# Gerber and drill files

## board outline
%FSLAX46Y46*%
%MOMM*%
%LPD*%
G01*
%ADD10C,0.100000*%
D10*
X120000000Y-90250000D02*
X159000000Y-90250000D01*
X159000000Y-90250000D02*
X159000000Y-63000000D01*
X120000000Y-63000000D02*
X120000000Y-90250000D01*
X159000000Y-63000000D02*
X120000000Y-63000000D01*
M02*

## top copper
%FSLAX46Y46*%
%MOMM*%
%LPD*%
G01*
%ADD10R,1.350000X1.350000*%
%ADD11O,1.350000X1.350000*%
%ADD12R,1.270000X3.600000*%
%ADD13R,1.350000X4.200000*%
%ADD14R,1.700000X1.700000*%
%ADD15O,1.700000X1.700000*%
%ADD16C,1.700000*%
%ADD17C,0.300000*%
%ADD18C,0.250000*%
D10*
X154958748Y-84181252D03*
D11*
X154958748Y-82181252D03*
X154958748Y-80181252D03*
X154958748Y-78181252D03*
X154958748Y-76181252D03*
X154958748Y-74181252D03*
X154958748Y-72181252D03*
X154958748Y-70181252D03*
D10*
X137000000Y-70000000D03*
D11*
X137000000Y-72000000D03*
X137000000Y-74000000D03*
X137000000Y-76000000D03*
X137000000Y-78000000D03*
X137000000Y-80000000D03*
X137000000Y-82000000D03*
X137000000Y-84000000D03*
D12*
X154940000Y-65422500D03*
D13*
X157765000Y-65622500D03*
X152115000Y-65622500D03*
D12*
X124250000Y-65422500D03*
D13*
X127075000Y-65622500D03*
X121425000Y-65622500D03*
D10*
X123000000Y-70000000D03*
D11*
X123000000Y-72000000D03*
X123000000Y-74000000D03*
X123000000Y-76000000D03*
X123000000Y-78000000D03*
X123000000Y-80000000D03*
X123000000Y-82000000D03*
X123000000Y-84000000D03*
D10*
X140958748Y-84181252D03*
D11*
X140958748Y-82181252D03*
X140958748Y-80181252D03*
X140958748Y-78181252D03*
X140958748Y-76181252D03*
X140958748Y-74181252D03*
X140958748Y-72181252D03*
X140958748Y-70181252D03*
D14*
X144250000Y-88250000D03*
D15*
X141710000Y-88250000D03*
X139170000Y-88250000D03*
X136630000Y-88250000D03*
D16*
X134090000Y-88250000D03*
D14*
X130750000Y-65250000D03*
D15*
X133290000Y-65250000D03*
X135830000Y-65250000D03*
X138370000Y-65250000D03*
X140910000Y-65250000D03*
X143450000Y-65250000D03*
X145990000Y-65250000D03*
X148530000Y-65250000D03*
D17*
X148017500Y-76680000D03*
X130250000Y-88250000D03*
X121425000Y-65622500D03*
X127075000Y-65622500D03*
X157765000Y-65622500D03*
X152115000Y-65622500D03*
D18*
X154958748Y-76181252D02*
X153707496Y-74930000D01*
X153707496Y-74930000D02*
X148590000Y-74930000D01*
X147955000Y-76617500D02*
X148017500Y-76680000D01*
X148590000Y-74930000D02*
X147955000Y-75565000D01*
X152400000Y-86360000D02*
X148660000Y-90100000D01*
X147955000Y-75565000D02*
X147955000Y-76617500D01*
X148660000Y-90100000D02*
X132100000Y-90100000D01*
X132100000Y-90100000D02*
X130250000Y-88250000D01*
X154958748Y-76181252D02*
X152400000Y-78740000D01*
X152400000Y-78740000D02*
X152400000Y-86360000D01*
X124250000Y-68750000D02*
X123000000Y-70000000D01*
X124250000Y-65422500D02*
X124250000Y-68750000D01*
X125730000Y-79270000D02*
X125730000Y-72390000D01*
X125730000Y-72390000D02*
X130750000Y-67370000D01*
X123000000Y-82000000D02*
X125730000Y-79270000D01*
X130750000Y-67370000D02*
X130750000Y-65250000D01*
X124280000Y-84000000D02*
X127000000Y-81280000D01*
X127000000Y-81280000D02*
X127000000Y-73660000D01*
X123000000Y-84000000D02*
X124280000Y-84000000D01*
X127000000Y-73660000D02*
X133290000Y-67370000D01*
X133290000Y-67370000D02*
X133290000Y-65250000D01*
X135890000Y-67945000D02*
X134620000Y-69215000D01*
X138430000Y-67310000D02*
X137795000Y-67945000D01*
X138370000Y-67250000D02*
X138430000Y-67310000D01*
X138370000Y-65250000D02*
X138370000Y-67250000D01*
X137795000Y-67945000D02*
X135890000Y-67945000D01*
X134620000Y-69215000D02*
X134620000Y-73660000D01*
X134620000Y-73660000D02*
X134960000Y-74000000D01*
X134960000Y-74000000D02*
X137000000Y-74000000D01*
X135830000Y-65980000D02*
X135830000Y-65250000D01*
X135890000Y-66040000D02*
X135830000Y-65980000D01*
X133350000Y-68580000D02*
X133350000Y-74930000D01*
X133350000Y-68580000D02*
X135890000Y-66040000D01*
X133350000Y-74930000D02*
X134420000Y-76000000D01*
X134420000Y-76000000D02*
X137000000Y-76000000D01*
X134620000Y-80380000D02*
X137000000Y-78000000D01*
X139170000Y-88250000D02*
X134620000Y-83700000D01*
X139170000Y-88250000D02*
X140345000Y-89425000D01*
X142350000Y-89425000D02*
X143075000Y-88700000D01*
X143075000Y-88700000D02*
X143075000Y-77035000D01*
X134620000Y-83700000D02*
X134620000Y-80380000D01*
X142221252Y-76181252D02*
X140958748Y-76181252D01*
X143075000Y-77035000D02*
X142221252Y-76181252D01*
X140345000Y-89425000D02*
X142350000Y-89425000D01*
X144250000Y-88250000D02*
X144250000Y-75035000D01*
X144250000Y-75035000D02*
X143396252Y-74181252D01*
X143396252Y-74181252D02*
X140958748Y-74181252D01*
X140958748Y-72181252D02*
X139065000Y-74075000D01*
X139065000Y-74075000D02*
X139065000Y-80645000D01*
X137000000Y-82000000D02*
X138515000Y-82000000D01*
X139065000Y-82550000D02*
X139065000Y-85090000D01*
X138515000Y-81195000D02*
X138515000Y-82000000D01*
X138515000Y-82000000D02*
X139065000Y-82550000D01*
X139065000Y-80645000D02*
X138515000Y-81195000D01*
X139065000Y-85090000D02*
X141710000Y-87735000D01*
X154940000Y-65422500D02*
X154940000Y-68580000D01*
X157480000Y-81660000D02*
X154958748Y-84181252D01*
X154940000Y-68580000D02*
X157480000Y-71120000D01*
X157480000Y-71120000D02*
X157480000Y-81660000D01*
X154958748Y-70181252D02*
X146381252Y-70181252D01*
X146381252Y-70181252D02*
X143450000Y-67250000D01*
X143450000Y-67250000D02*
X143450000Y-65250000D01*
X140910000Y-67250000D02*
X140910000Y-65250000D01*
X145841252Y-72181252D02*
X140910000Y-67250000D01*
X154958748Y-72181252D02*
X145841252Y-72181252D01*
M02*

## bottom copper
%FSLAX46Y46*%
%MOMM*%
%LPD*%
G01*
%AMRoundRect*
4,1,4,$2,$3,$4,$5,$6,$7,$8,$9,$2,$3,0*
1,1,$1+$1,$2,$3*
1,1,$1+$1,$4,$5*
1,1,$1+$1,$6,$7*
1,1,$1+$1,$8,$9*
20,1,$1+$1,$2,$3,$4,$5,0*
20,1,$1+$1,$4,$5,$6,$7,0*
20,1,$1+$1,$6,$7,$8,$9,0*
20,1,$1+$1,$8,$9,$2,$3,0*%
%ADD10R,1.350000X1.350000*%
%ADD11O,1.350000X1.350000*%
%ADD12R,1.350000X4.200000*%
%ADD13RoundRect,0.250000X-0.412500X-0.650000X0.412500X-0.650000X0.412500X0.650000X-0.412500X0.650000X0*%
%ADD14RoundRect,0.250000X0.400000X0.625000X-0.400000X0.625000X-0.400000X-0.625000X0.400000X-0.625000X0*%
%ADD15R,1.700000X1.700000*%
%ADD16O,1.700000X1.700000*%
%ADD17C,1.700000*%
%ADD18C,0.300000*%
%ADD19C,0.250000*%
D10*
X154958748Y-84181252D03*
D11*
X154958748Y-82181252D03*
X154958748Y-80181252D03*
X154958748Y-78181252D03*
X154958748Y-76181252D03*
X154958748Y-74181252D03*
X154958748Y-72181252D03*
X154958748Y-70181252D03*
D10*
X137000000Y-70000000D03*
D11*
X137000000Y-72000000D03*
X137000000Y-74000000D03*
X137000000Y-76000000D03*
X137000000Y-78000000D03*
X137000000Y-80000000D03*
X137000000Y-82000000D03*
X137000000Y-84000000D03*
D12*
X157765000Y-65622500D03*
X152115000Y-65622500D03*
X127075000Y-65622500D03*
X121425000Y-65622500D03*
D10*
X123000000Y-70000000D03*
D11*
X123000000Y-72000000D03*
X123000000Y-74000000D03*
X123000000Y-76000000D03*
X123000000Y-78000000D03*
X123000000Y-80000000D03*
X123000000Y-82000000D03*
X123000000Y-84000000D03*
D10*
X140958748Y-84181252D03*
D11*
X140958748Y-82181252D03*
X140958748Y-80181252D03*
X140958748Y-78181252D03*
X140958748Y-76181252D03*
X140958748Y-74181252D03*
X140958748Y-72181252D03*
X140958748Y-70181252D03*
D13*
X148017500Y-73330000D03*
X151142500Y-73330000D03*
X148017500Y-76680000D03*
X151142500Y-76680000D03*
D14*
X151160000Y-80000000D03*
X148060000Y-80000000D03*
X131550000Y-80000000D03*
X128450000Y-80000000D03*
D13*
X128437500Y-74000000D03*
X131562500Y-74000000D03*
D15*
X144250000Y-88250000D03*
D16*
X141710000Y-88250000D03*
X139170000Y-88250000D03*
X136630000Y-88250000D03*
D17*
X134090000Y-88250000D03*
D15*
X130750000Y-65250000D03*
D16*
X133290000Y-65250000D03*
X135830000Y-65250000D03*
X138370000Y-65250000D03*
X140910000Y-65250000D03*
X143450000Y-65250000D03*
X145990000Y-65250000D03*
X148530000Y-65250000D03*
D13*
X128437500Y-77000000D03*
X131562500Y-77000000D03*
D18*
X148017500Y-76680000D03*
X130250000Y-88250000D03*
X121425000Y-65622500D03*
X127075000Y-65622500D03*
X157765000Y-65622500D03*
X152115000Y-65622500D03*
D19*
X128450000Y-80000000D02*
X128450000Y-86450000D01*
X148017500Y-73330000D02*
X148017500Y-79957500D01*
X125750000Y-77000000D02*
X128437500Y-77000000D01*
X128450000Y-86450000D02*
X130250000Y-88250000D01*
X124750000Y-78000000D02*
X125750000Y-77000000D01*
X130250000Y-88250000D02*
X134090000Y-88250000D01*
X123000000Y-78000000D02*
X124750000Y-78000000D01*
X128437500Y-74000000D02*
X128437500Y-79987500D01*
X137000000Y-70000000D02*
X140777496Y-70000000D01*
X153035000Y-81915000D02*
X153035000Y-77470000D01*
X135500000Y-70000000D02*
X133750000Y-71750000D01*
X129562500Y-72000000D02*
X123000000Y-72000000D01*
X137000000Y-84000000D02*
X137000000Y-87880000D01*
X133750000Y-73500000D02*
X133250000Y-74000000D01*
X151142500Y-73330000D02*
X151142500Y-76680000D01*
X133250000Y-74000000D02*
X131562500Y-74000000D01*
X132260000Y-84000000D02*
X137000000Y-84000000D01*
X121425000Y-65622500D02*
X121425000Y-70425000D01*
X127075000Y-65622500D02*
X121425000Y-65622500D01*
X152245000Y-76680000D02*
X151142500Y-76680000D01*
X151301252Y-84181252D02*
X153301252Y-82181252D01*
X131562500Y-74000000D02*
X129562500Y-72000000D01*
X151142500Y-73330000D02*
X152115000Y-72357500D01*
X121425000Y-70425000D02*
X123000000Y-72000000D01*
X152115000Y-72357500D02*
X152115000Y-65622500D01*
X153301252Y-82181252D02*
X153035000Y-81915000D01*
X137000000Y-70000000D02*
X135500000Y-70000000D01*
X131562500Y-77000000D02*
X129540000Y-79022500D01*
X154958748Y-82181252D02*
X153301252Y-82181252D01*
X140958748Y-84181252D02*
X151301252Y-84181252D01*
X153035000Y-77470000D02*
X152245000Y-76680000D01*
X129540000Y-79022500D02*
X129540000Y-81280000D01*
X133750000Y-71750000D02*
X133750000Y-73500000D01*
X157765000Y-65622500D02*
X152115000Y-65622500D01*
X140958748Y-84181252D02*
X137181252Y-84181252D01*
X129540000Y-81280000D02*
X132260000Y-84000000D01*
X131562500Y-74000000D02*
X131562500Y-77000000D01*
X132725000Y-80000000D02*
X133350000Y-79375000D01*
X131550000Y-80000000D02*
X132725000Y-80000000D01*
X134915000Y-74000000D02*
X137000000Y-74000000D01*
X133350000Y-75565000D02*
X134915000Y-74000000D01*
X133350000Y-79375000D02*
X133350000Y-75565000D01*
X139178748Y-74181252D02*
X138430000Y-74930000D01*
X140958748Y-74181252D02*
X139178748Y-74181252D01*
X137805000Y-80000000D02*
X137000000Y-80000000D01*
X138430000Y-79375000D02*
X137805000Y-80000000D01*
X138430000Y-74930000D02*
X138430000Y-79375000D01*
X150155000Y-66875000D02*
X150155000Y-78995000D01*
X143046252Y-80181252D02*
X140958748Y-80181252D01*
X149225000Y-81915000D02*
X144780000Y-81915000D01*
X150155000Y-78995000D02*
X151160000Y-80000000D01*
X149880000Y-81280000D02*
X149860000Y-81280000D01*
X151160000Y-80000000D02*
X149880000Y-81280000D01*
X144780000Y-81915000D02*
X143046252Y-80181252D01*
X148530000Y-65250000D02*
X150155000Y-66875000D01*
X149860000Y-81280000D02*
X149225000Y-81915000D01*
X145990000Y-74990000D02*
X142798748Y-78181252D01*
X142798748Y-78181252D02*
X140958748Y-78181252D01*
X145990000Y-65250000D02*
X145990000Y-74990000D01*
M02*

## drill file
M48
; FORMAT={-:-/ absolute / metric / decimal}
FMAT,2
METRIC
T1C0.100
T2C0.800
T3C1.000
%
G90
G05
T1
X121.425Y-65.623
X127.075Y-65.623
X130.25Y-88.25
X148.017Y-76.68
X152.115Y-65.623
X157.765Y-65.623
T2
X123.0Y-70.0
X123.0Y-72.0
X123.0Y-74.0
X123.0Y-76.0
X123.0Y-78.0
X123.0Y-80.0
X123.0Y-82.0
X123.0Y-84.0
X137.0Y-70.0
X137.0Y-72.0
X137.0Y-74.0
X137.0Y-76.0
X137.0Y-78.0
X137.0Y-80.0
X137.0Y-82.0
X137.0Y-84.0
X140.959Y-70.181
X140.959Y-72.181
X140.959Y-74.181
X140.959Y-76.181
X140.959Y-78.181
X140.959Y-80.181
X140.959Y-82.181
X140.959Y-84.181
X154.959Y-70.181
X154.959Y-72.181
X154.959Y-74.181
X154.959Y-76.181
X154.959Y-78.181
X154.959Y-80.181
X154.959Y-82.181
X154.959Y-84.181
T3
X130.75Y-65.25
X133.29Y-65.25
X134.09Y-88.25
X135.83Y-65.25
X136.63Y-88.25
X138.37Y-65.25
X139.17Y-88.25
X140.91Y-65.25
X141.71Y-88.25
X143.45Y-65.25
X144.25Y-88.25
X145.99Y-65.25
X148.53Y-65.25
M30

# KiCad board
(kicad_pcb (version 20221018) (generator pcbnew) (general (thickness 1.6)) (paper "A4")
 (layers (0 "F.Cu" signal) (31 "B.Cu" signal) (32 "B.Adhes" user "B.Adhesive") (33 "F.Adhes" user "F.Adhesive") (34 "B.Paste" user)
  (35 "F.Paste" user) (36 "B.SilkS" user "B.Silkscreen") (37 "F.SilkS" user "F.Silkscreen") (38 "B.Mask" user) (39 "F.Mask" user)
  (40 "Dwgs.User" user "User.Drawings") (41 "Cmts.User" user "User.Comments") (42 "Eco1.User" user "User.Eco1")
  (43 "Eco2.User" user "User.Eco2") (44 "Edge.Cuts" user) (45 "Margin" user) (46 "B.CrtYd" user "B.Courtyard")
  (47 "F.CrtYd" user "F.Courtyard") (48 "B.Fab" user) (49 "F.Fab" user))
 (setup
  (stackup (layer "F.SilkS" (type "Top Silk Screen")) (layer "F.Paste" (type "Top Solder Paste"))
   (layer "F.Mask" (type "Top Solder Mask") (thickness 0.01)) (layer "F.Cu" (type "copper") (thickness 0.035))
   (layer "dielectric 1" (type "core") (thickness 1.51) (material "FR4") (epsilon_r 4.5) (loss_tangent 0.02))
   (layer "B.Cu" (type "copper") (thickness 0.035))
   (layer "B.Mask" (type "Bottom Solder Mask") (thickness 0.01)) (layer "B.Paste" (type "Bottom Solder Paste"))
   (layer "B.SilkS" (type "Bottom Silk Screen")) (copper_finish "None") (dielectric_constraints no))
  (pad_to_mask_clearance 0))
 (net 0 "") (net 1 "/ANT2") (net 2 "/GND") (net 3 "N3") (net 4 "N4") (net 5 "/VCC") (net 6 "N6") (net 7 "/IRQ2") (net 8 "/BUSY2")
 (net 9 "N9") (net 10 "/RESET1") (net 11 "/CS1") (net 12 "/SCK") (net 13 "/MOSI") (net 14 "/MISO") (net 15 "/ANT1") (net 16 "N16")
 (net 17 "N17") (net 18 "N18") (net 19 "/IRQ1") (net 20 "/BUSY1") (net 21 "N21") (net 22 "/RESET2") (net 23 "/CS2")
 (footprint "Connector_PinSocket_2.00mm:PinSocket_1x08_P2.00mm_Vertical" (layer "F.Cu") (at 154.958748 84.181252 180)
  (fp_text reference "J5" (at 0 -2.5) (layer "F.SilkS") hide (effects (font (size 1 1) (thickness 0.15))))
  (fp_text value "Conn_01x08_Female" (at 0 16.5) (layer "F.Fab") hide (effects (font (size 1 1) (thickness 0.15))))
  (pad "1" thru_hole rect (at 0 0 180) (size 1.35 1.35) (drill 0.8) (layers "*.Cu" "*.Mask") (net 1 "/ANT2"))
  (pad "2" thru_hole oval (at 0 2 180) (size 1.35 1.35) (drill 0.8) (layers "*.Cu" "*.Mask") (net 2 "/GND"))
  (pad "3" thru_hole oval (at 0 4 180) (size 1.35 1.35) (drill 0.8) (layers "*.Cu" "*.Mask") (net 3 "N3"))
  (pad "4" thru_hole oval (at 0 6 180) (size 1.35 1.35) (drill 0.8) (layers "*.Cu" "*.Mask") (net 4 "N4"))
  (pad "5" thru_hole oval (at 0 8 180) (size 1.35 1.35) (drill 0.8) (layers "*.Cu" "*.Mask") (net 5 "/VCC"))
  (pad "6" thru_hole oval (at 0 10 180) (size 1.35 1.35) (drill 0.8) (layers "*.Cu" "*.Mask") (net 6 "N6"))
  (pad "7" thru_hole oval (at 0 12 180) (size 1.35 1.35) (drill 0.8) (layers "*.Cu" "*.Mask") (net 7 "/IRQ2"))
  (pad "8" thru_hole oval (at 0 14 180) (size 1.35 1.35) (drill 0.8) (layers "*.Cu" "*.Mask") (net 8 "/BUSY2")))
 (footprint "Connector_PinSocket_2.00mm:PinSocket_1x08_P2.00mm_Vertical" (layer "F.Cu") (at 137 70)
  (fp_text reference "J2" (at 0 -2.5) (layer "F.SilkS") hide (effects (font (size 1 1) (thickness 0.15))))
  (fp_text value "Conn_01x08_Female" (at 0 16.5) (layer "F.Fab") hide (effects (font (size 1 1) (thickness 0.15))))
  (pad "1" thru_hole rect (at 0 0) (size 1.35 1.35) (drill 0.8) (layers "*.Cu" "*.Mask") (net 2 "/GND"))
  (pad "2" thru_hole oval (at 0 2) (size 1.35 1.35) (drill 0.8) (layers "*.Cu" "*.Mask") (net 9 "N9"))
  (pad "3" thru_hole oval (at 0 4) (size 1.35 1.35) (drill 0.8) (layers "*.Cu" "*.Mask") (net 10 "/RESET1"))
  (pad "4" thru_hole oval (at 0 6) (size 1.35 1.35) (drill 0.8) (layers "*.Cu" "*.Mask") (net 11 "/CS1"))
  (pad "5" thru_hole oval (at 0 8) (size 1.35 1.35) (drill 0.8) (layers "*.Cu" "*.Mask") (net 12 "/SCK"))
  (pad "6" thru_hole oval (at 0 10) (size 1.35 1.35) (drill 0.8) (layers "*.Cu" "*.Mask") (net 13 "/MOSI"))
  (pad "7" thru_hole oval (at 0 12) (size 1.35 1.35) (drill 0.8) (layers "*.Cu" "*.Mask") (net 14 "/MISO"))
  (pad "8" thru_hole oval (at 0 14) (size 1.35 1.35) (drill 0.8) (layers "*.Cu" "*.Mask") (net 2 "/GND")))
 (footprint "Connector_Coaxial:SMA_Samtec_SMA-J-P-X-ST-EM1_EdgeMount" (layer "F.Cu") (at 154.94 65.6225 180)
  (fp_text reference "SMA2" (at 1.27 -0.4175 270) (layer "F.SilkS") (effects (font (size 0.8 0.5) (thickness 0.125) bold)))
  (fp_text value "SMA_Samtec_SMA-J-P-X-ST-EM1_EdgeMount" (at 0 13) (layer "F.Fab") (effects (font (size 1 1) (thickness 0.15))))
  (pad "1" smd rect (at -2.825 0 180) (size 1.35 4.2) (layers "B.Cu" "B.Paste" "B.Mask") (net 2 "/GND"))
  (pad "1" smd rect (at 0 0.2 180) (size 1.27 3.6) (layers "F.Cu" "F.Paste" "F.Mask") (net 1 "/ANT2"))
  (pad "1" smd rect (at 2.825 0 180) (size 1.35 4.2) (layers "B.Cu" "B.Paste" "B.Mask") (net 2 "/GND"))
  (pad "2" smd rect (at -2.825 0 180) (size 1.35 4.2) (layers "F.Cu" "F.Paste" "F.Mask") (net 2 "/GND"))
  (pad "2" smd rect (at 2.825 0 180) (size 1.35 4.2) (layers "F.Cu" "F.Paste" "F.Mask") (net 2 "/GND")))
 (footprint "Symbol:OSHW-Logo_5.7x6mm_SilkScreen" (layer "F.Cu") (at 149 86.5)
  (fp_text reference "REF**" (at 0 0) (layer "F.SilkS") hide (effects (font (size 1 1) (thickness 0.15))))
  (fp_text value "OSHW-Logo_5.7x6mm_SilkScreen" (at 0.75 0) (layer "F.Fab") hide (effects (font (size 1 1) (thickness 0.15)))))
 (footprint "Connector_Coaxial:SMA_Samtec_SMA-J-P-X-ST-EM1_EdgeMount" (layer "F.Cu") (at 124.25 65.6225 180)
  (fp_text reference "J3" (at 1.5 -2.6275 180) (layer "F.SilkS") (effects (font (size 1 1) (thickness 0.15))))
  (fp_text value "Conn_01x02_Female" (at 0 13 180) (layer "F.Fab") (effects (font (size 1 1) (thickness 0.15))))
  (pad "1" smd rect (at -2.825 0 180) (size 1.35 4.2) (layers "B.Cu" "B.Paste" "B.Mask") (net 2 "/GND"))
  (pad "1" smd rect (at 0 0.2 180) (size 1.27 3.6) (layers "F.Cu" "F.Paste" "F.Mask") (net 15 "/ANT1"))
  (pad "1" smd rect (at 2.825 0 180) (size 1.35 4.2) (layers "B.Cu" "B.Paste" "B.Mask") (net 2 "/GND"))
  (pad "2" smd rect (at -2.825 0 180) (size 1.35 4.2) (layers "F.Cu" "F.Paste" "F.Mask") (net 2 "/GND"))
  (pad "2" smd rect (at 2.825 0 180) (size 1.35 4.2) (layers "F.Cu" "F.Paste" "F.Mask") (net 2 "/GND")))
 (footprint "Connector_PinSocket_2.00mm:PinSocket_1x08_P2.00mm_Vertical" (layer "F.Cu") (at 123 70)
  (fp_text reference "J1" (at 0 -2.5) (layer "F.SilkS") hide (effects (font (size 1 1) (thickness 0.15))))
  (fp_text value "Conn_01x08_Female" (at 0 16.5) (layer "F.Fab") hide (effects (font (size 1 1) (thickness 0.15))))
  (pad "1" thru_hole rect (at 0 0) (size 1.35 1.35) (drill 0.8) (layers "*.Cu" "*.Mask") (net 15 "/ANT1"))
  (pad "2" thru_hole oval (at 0 2) (size 1.35 1.35) (drill 0.8) (layers "*.Cu" "*.Mask") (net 2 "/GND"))
  (pad "3" thru_hole oval (at 0 4) (size 1.35 1.35) (drill 0.8) (layers "*.Cu" "*.Mask") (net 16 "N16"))
  (pad "4" thru_hole oval (at 0 6) (size 1.35 1.35) (drill 0.8) (layers "*.Cu" "*.Mask") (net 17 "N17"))
  (pad "5" thru_hole oval (at 0 8) (size 1.35 1.35) (drill 0.8) (layers "*.Cu" "*.Mask") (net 5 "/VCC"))
  (pad "6" thru_hole oval (at 0 10) (size 1.35 1.35) (drill 0.8) (layers "*.Cu" "*.Mask") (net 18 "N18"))
  (pad "7" thru_hole oval (at 0 12) (size 1.35 1.35) (drill 0.8) (layers "*.Cu" "*.Mask") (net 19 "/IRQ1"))
  (pad "8" thru_hole oval (at 0 14) (size 1.35 1.35) (drill 0.8) (layers "*.Cu" "*.Mask") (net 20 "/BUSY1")))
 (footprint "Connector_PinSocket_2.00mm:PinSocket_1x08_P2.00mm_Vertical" (layer "F.Cu") (at 140.958748 84.181252 180)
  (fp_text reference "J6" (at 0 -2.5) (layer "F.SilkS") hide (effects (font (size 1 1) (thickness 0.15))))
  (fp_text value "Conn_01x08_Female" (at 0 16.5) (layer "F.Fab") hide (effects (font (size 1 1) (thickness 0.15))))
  (pad "1" thru_hole rect (at 0 0 180) (size 1.35 1.35) (drill 0.8) (layers "*.Cu" "*.Mask") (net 2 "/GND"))
  (pad "2" thru_hole oval (at 0 2 180) (size 1.35 1.35) (drill 0.8) (layers "*.Cu" "*.Mask") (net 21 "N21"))
  (pad "3" thru_hole oval (at 0 4 180) (size 1.35 1.35) (drill 0.8) (layers "*.Cu" "*.Mask") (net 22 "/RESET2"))
  (pad "4" thru_hole oval (at 0 6 180) (size 1.35 1.35) (drill 0.8) (layers "*.Cu" "*.Mask") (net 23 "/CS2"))
  (pad "5" thru_hole oval (at 0 8 180) (size 1.35 1.35) (drill 0.8) (layers "*.Cu" "*.Mask") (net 12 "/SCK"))
  (pad "6" thru_hole oval (at 0 10 180) (size 1.35 1.35) (drill 0.8) (layers "*.Cu" "*.Mask") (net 13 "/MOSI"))
  (pad "7" thru_hole oval (at 0 12 180) (size 1.35 1.35) (drill 0.8) (layers "*.Cu" "*.Mask") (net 14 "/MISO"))
  (pad "8" thru_hole oval (at 0 14 180) (size 1.35 1.35) (drill 0.8) (layers "*.Cu" "*.Mask") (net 2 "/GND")))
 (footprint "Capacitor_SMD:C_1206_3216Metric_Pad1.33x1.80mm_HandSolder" (layer "B.Cu") (at 149.58 73.33)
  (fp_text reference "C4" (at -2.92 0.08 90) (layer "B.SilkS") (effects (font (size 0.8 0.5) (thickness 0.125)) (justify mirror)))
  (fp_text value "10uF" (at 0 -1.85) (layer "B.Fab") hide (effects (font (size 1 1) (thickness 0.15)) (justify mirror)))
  (pad "1" smd roundrect (at -1.5625 0) (size 1.325 1.8) (layers "B.Cu" "B.Paste" "B.Mask") (roundrect_rratio 0.1886792453) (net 5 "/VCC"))
  (pad "2" smd roundrect (at 1.5625 0) (size 1.325 1.8) (layers "B.Cu" "B.Paste" "B.Mask") (roundrect_rratio 0.1886792453) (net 2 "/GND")))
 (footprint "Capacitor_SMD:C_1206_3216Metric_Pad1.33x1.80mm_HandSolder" (layer "B.Cu") (at 149.58 76.68)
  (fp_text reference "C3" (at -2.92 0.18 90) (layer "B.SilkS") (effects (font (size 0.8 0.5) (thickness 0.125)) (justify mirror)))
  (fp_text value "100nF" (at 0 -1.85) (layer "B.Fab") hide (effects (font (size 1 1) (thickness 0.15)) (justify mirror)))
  (pad "1" smd roundrect (at -1.5625 0) (size 1.325 1.8) (layers "B.Cu" "B.Paste" "B.Mask") (roundrect_rratio 0.1886792453) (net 5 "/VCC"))
  (pad "2" smd roundrect (at 1.5625 0) (size 1.325 1.8) (layers "B.Cu" "B.Paste" "B.Mask") (roundrect_rratio 0.1886792453) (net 2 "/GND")))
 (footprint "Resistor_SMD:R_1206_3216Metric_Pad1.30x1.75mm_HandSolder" (layer "B.Cu") (at 149.61 80 180)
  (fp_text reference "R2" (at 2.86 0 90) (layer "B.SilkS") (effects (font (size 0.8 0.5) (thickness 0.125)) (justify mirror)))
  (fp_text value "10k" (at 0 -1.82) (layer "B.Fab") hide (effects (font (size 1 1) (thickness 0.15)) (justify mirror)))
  (pad "1" smd roundrect (at -1.55 0 180) (size 1.3 1.75) (layers "B.Cu" "B.Paste" "B.Mask") (roundrect_rratio 0.1923076923)
   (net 22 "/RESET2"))
  (pad "2" smd roundrect (at 1.55 0 180) (size 1.3 1.75) (layers "B.Cu" "B.Paste" "B.Mask") (roundrect_rratio 0.1923076923) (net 5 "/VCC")))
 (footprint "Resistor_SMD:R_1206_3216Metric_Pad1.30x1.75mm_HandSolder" (layer "B.Cu") (at 130 80 180)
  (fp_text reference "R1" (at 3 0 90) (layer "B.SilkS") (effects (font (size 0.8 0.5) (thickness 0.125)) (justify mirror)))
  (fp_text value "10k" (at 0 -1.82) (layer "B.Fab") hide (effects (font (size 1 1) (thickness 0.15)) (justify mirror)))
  (pad "1" smd roundrect (at -1.55 0 180) (size 1.3 1.75) (layers "B.Cu" "B.Paste" "B.Mask") (roundrect_rratio 0.1923076923)
   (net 10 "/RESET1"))
  (pad "2" smd roundrect (at 1.55 0 180) (size 1.3 1.75) (layers "B.Cu" "B.Paste" "B.Mask") (roundrect_rratio 0.1923076923) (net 5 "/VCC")))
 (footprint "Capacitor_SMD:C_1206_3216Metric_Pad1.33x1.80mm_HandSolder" (layer "B.Cu") (at 130 74)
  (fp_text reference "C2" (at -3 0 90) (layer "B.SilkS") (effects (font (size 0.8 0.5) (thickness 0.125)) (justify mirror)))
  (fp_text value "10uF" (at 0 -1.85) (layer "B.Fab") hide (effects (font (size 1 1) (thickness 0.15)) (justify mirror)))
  (pad "1" smd roundrect (at -1.5625 0) (size 1.325 1.8) (layers "B.Cu" "B.Paste" "B.Mask") (roundrect_rratio 0.1886792453) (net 5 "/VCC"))
  (pad "2" smd roundrect (at 1.5625 0) (size 1.325 1.8) (layers "B.Cu" "B.Paste" "B.Mask") (roundrect_rratio 0.1886792453) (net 2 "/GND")))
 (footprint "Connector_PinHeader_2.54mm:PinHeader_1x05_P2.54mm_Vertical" (layer "B.Cu") (at 144.25 88.25 90)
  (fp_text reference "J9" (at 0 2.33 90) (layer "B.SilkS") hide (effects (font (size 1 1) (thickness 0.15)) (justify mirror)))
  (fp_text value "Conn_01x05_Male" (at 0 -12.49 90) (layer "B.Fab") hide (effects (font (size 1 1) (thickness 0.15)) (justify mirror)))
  (pad "1" thru_hole rect (at 0 0 90) (size 1.7 1.7) (drill 1) (layers "*.Cu" "*.Mask") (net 13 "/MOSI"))
  (pad "2" thru_hole oval (at 0 -2.54 90) (size 1.7 1.7) (drill 1) (layers "*.Cu" "*.Mask") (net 14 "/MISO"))
  (pad "3" thru_hole oval (at 0 -5.08 90) (size 1.7 1.7) (drill 1) (layers "*.Cu" "*.Mask") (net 12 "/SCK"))
  (pad "4" thru_hole oval (at 0 -7.62 90) (size 1.7 1.7) (drill 1) (layers "*.Cu" "*.Mask") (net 2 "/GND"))
  (pad "5" thru_hole circle (at 0 -10.16 90) (size 1.7 1.7) (drill 1) (layers "*.Cu" "*.Mask") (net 5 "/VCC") (zone_connect 2)))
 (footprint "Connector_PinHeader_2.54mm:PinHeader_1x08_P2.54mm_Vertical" (layer "B.Cu") (at 130.75 65.25 -90)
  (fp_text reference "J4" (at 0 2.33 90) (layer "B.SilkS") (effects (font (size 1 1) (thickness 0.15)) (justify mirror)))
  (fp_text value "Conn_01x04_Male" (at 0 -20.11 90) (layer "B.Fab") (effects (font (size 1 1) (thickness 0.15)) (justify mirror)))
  (pad "1" thru_hole rect (at 0 0 270) (size 1.7 1.7) (drill 1) (layers "*.Cu" "*.Mask") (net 19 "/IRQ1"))
  (pad "2" thru_hole oval (at 0 -2.54 270) (size 1.7 1.7) (drill 1) (layers "*.Cu" "*.Mask") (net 20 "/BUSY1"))
  (pad "3" thru_hole oval (at 0 -5.08 270) (size 1.7 1.7) (drill 1) (layers "*.Cu" "*.Mask") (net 11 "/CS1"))
  (pad "4" thru_hole oval (at 0 -7.62 270) (size 1.7 1.7) (drill 1) (layers "*.Cu" "*.Mask") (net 10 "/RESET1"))
  (pad "5" thru_hole oval (at 0 -10.16 270) (size 1.7 1.7) (drill 1) (layers "*.Cu" "*.Mask") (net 7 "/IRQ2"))
  (pad "6" thru_hole oval (at 0 -12.7 270) (size 1.7 1.7) (drill 1) (layers "*.Cu" "*.Mask") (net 8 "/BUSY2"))
  (pad "7" thru_hole oval (at 0 -15.24 270) (size 1.7 1.7) (drill 1) (layers "*.Cu" "*.Mask") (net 23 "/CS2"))
  (pad "8" thru_hole oval (at 0 -17.78 270) (size 1.7 1.7) (drill 1) (layers "*.Cu" "*.Mask") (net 22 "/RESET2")))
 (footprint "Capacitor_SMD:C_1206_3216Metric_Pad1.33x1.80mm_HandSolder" (layer "B.Cu") (at 130 77)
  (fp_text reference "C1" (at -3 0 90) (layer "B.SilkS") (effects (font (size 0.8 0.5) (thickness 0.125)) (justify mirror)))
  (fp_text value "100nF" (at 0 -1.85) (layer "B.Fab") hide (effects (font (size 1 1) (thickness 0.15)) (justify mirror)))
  (pad "1" smd roundrect (at -1.5625 0) (size 1.325 1.8) (layers "B.Cu" "B.Paste" "B.Mask") (roundrect_rratio 0.1886792453) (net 5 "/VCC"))
  (pad "2" smd roundrect (at 1.5625 0) (size 1.325 1.8) (layers "B.Cu" "B.Paste" "B.Mask") (roundrect_rratio 0.1886792453) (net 2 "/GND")))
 (gr_line (start 120 90.25) (end 159 90.25) (stroke (width 0.1) (type solid)) (layer "Edge.Cuts"))
 (gr_line (start 159 90.25) (end 159 63) (stroke (width 0.1) (type solid)) (layer "Edge.Cuts"))
 (gr_line (start 120 63) (end 120 90.25) (stroke (width 0.1) (type solid)) (layer "Edge.Cuts"))
 (gr_line (start 159 63) (end 120 63) (stroke (width 0.1) (type solid)) (layer "Edge.Cuts"))
 (segment (start 154.958748 76.181252) (end 153.707496 74.93) (width 0.25) (layer "F.Cu") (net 5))
 (segment (start 153.707496 74.93) (end 148.59 74.93) (width 0.25) (layer "F.Cu") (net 5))
 (segment (start 147.955 76.6175) (end 148.0175 76.68) (width 0.25) (layer "F.Cu") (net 5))
 (segment (start 148.59 74.93) (end 147.955 75.565) (width 0.25) (layer "F.Cu") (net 5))
 (segment (start 152.4 86.36) (end 148.66 90.1) (width 0.25) (layer "F.Cu") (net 5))
 (segment (start 147.955 75.565) (end 147.955 76.6175) (width 0.25) (layer "F.Cu") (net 5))
 (segment (start 148.66 90.1) (end 132.1 90.1) (width 0.25) (layer "F.Cu") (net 5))
 (segment (start 132.1 90.1) (end 130.25 88.25) (width 0.25) (layer "F.Cu") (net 5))
 (segment (start 154.958748 76.181252) (end 152.4 78.74) (width 0.25) (layer "F.Cu") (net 5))
 (segment (start 152.4 78.74) (end 152.4 86.36) (width 0.25) (layer "F.Cu") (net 5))
 (via micro (at 148.0175 76.68) (size 0.3) (drill 0.1) (layers "F.Cu" "B.Cu") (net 5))
 (via micro (at 130.25 88.25) (size 0.3) (drill 0.1) (layers "F.Cu" "B.Cu") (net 5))
 (segment (start 128.45 80) (end 128.45 86.45) (width 0.25) (layer "B.Cu") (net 5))
 (segment (start 148.0175 73.33) (end 148.0175 79.9575) (width 0.25) (layer "B.Cu") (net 5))
 (segment (start 125.75 77) (end 128.4375 77) (width 0.25) (layer "B.Cu") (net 5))
 (segment (start 128.45 86.45) (end 130.25 88.25) (width 0.25) (layer "B.Cu") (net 5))
 (segment (start 124.75 78) (end 125.75 77) (width 0.25) (layer "B.Cu") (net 5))
 (segment (start 130.25 88.25) (end 134.09 88.25) (width 0.25) (layer "B.Cu") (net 5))
 (segment (start 123 78) (end 124.75 78) (width 0.25) (layer "B.Cu") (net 5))
 (segment (start 128.4375 74) (end 128.4375 79.9875) (width 0.25) (layer "B.Cu") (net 5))
 (via micro (at 121.425 65.6225) (size 0.3) (drill 0.1) (layers "F.Cu" "B.Cu") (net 2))
 (via micro (at 127.075 65.6225) (size 0.3) (drill 0.1) (layers "F.Cu" "B.Cu") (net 2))
 (via micro (at 157.765 65.6225) (size 0.3) (drill 0.1) (layers "F.Cu" "B.Cu") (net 2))
 (via micro (at 152.115 65.6225) (size 0.3) (drill 0.1) (layers "F.Cu" "B.Cu") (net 2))
 (segment (start 137 70) (end 140.777496 70) (width 0.25) (layer "B.Cu") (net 2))
 (segment (start 153.035 81.915) (end 153.035 77.47) (width 0.25) (layer "B.Cu") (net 2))
 (segment (start 135.5 70) (end 133.75 71.75) (width 0.25) (layer "B.Cu") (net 2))
 (segment (start 129.5625 72) (end 123 72) (width 0.25) (layer "B.Cu") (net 2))
 (segment (start 137 84) (end 137 87.88) (width 0.25) (layer "B.Cu") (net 2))
 (segment (start 133.75 73.5) (end 133.25 74) (width 0.25) (layer "B.Cu") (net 2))
 (segment (start 151.1425 73.33) (end 151.1425 76.68) (width 0.25) (layer "B.Cu") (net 2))
 (segment (start 133.25 74) (end 131.5625 74) (width 0.25) (layer "B.Cu") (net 2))
 (segment (start 132.26 84) (end 137 84) (width 0.25) (layer "B.Cu") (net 2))
 (segment (start 121.425 65.6225) (end 121.425 70.425) (width 0.25) (layer "B.Cu") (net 2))
 (segment (start 127.075 65.6225) (end 121.425 65.6225) (width 0.25) (layer "B.Cu") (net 2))
 (segment (start 152.245 76.68) (end 151.1425 76.68) (width 0.25) (layer "B.Cu") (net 2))
 (segment (start 151.301252 84.181252) (end 153.301252 82.181252) (width 0.25) (layer "B.Cu") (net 2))
 (segment (start 131.5625 74) (end 129.5625 72) (width 0.25) (layer "B.Cu") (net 2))
 (segment (start 151.1425 73.33) (end 152.115 72.3575) (width 0.25) (layer "B.Cu") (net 2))
 (segment (start 121.425 70.425) (end 123 72) (width 0.25) (layer "B.Cu") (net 2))
 (segment (start 152.115 72.3575) (end 152.115 65.6225) (width 0.25) (layer "B.Cu") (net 2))
 (segment (start 153.301252 82.181252) (end 153.035 81.915) (width 0.25) (layer "B.Cu") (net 2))
 (segment (start 137 70) (end 135.5 70) (width 0.25) (layer "B.Cu") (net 2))
 (segment (start 131.5625 77) (end 129.54 79.0225) (width 0.25) (layer "B.Cu") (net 2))
 (segment (start 154.958748 82.181252) (end 153.301252 82.181252) (width 0.25) (layer "B.Cu") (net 2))
 (segment (start 140.958748 84.181252) (end 151.301252 84.181252) (width 0.25) (layer "B.Cu") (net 2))
 (segment (start 153.035 77.47) (end 152.245 76.68) (width 0.25) (layer "B.Cu") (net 2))
 (segment (start 129.54 79.0225) (end 129.54 81.28) (width 0.25) (layer "B.Cu") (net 2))
 (segment (start 133.75 71.75) (end 133.75 73.5) (width 0.25) (layer "B.Cu") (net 2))
 (segment (start 157.765 65.6225) (end 152.115 65.6225) (width 0.25) (layer "B.Cu") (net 2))
 (segment (start 140.958748 84.181252) (end 137.181252 84.181252) (width 0.25) (layer "B.Cu") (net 2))
 (segment (start 129.54 81.28) (end 132.26 84) (width 0.25) (layer "B.Cu") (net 2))
 (segment (start 131.5625 74) (end 131.5625 77) (width 0.25) (layer "B.Cu") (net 2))
 (segment (start 124.25 68.75) (end 123 70) (width 0.25) (layer "F.Cu") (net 15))
 (segment (start 124.25 65.4225) (end 124.25 68.75) (width 0.25) (layer "F.Cu") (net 15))
 (segment (start 125.73 79.27) (end 125.73 72.39) (width 0.25) (layer "F.Cu") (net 19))
 (segment (start 125.73 72.39) (end 130.75 67.37) (width 0.25) (layer "F.Cu") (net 19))
 (segment (start 123 82) (end 125.73 79.27) (width 0.25) (layer "F.Cu") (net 19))
 (segment (start 130.75 67.37) (end 130.75 65.25) (width 0.25) (layer "F.Cu") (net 19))
 (segment (start 124.28 84) (end 127 81.28) (width 0.25) (layer "F.Cu") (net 20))
 (segment (start 127 81.28) (end 127 73.66) (width 0.25) (layer "F.Cu") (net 20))
 (segment (start 123 84) (end 124.28 84) (width 0.25) (layer "F.Cu") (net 20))
 (segment (start 127 73.66) (end 133.29 67.37) (width 0.25) (layer "F.Cu") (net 20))
 (segment (start 133.29 67.37) (end 133.29 65.25) (width 0.25) (layer "F.Cu") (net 20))
 (segment (start 135.89 67.945) (end 134.62 69.215) (width 0.25) (layer "F.Cu") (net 10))
 (segment (start 138.43 67.31) (end 137.795 67.945) (width 0.25) (layer "F.Cu") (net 10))
 (segment (start 138.37 67.25) (end 138.43 67.31) (width 0.25) (layer "F.Cu") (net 10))
 (segment (start 138.37 65.25) (end 138.37 67.25) (width 0.25) (layer "F.Cu") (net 10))
 (segment (start 137.795 67.945) (end 135.89 67.945) (width 0.25) (layer "F.Cu") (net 10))
 (segment (start 134.62 69.215) (end 134.62 73.66) (width 0.25) (layer "F.Cu") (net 10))
 (segment (start 134.62 73.66) (end 134.96 74) (width 0.25) (layer "F.Cu") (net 10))
 (segment (start 134.96 74) (end 137 74) (width 0.25) (layer "F.Cu") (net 10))
 (segment (start 132.725 80) (end 133.35 79.375) (width 0.25) (layer "B.Cu") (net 10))
 (segment (start 131.55 80) (end 132.725 80) (width 0.25) (layer "B.Cu") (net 10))
 (segment (start 134.915 74) (end 137 74) (width 0.25) (layer "B.Cu") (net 10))
 (segment (start 133.35 75.565) (end 134.915 74) (width 0.25) (layer "B.Cu") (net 10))
 (segment (start 133.35 79.375) (end 133.35 75.565) (width 0.25) (layer "B.Cu") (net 10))
 (segment (start 135.83 65.98) (end 135.83 65.25) (width 0.25) (layer "F.Cu") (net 11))
 (segment (start 135.89 66.04) (end 135.83 65.98) (width 0.25) (layer "F.Cu") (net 11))
 (segment (start 133.35 68.58) (end 133.35 74.93) (width 0.25) (layer "F.Cu") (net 11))
 (segment (start 133.35 68.58) (end 135.89 66.04) (width 0.25) (layer "F.Cu") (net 11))
 (segment (start 133.35 74.93) (end 134.42 76) (width 0.25) (layer "F.Cu") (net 11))
 (segment (start 134.42 76) (end 137 76) (width 0.25) (layer "F.Cu") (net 11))
 (segment (start 134.62 80.38) (end 137 78) (width 0.25) (layer "F.Cu") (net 12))
 (segment (start 139.17 88.25) (end 134.62 83.7) (width 0.25) (layer "F.Cu") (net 12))
 (segment (start 139.17 88.25) (end 140.345 89.425) (width 0.25) (layer "F.Cu") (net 12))
 (segment (start 142.35 89.425) (end 143.075 88.7) (width 0.25) (layer "F.Cu") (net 12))
 (segment (start 143.075 88.7) (end 143.075 77.035) (width 0.25) (layer "F.Cu") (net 12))
 (segment (start 134.62 83.7) (end 134.62 80.38) (width 0.25) (layer "F.Cu") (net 12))
 (segment (start 142.221252 76.181252) (end 140.958748 76.181252) (width 0.25) (layer "F.Cu") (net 12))
 (segment (start 143.075 77.035) (end 142.221252 76.181252) (width 0.25) (layer "F.Cu") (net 12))
 (segment (start 140.345 89.425) (end 142.35 89.425) (width 0.25) (layer "F.Cu") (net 12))
 (segment (start 144.25 88.25) (end 144.25 75.035) (width 0.25) (layer "F.Cu") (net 13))
 (segment (start 144.25 75.035) (end 143.396252 74.181252) (width 0.25) (layer "F.Cu") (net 13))
 (segment (start 143.396252 74.181252) (end 140.958748 74.181252) (width 0.25) (layer "F.Cu") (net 13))
 (segment (start 139.178748 74.181252) (end 138.43 74.93) (width 0.25) (layer "B.Cu") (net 13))
 (segment (start 140.958748 74.181252) (end 139.178748 74.181252) (width 0.25) (layer "B.Cu") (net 13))
 (segment (start 137.805 80) (end 137 80) (width 0.25) (layer "B.Cu") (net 13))
 (segment (start 138.43 79.375) (end 137.805 80) (width 0.25) (layer "B.Cu") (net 13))
 (segment (start 138.43 74.93) (end 138.43 79.375) (width 0.25) (layer "B.Cu") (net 13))
 (segment (start 140.958748 72.181252) (end 139.065 74.075) (width 0.25) (layer "F.Cu") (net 14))
 (segment (start 139.065 74.075) (end 139.065 80.645) (width 0.25) (layer "F.Cu") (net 14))
 (segment (start 137 82) (end 138.515 82) (width 0.25) (layer "F.Cu") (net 14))
 (segment (start 139.065 82.55) (end 139.065 85.09) (width 0.25) (layer "F.Cu") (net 14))
 (segment (start 138.515 81.195) (end 138.515 82) (width 0.25) (layer "F.Cu") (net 14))
 (segment (start 138.515 82) (end 139.065 82.55) (width 0.25) (layer "F.Cu") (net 14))
 (segment (start 139.065 80.645) (end 138.515 81.195) (width 0.25) (layer "F.Cu") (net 14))
 (segment (start 139.065 85.09) (end 141.71 87.735) (width 0.25) (layer "F.Cu") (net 14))
 (segment (start 154.94 65.4225) (end 154.94 68.58) (width 0.25) (layer "F.Cu") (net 1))
 (segment (start 157.48 81.66) (end 154.958748 84.181252) (width 0.25) (layer "F.Cu") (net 1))
 (segment (start 154.94 68.58) (end 157.48 71.12) (width 0.25) (layer "F.Cu") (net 1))
 (segment (start 157.48 71.12) (end 157.48 81.66) (width 0.25) (layer "F.Cu") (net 1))
 (segment (start 154.958748 70.181252) (end 146.381252 70.181252) (width 0.25) (layer "F.Cu") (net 8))
 (segment (start 146.381252 70.181252) (end 143.45 67.25) (width 0.25) (layer "F.Cu") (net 8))
 (segment (start 143.45 67.25) (end 143.45 65.25) (width 0.25) (layer "F.Cu") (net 8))
 (segment (start 150.155 66.875) (end 150.155 78.995) (width 0.25) (layer "B.Cu") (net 22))
 (segment (start 143.046252 80.181252) (end 140.958748 80.181252) (width 0.25) (layer "B.Cu") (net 22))
 (segment (start 149.225 81.915) (end 144.78 81.915) (width 0.25) (layer "B.Cu") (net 22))
 (segment (start 150.155 78.995) (end 151.16 80) (width 0.25) (layer "B.Cu") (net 22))
 (segment (start 149.88 81.28) (end 149.86 81.28) (width 0.25) (layer "B.Cu") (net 22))
 (segment (start 151.16 80) (end 149.88 81.28) (width 0.25) (layer "B.Cu") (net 22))
 (segment (start 144.78 81.915) (end 143.046252 80.181252) (width 0.25) (layer "B.Cu") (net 22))
 (segment (start 148.53 65.25) (end 150.155 66.875) (width 0.25) (layer "B.Cu") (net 22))
 (segment (start 149.86 81.28) (end 149.225 81.915) (width 0.25) (layer "B.Cu") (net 22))
 (segment (start 145.99 74.99) (end 142.798748 78.181252) (width 0.25) (layer "B.Cu") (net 23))
 (segment (start 142.798748 78.181252) (end 140.958748 78.181252) (width 0.25) (layer "B.Cu") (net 23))
 (segment (start 145.99 65.25) (end 145.99 74.99) (width 0.25) (layer "B.Cu") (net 23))
 (segment (start 140.91 67.25) (end 140.91 65.25) (width 0.25) (layer "F.Cu") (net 7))
 (segment (start 145.841252 72.181252) (end 140.91 67.25) (width 0.25) (layer "F.Cu") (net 7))
 (segment (start 154.958748 72.181252) (end 145.841252 72.181252) (width 0.25) (layer "F.Cu") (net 7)))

